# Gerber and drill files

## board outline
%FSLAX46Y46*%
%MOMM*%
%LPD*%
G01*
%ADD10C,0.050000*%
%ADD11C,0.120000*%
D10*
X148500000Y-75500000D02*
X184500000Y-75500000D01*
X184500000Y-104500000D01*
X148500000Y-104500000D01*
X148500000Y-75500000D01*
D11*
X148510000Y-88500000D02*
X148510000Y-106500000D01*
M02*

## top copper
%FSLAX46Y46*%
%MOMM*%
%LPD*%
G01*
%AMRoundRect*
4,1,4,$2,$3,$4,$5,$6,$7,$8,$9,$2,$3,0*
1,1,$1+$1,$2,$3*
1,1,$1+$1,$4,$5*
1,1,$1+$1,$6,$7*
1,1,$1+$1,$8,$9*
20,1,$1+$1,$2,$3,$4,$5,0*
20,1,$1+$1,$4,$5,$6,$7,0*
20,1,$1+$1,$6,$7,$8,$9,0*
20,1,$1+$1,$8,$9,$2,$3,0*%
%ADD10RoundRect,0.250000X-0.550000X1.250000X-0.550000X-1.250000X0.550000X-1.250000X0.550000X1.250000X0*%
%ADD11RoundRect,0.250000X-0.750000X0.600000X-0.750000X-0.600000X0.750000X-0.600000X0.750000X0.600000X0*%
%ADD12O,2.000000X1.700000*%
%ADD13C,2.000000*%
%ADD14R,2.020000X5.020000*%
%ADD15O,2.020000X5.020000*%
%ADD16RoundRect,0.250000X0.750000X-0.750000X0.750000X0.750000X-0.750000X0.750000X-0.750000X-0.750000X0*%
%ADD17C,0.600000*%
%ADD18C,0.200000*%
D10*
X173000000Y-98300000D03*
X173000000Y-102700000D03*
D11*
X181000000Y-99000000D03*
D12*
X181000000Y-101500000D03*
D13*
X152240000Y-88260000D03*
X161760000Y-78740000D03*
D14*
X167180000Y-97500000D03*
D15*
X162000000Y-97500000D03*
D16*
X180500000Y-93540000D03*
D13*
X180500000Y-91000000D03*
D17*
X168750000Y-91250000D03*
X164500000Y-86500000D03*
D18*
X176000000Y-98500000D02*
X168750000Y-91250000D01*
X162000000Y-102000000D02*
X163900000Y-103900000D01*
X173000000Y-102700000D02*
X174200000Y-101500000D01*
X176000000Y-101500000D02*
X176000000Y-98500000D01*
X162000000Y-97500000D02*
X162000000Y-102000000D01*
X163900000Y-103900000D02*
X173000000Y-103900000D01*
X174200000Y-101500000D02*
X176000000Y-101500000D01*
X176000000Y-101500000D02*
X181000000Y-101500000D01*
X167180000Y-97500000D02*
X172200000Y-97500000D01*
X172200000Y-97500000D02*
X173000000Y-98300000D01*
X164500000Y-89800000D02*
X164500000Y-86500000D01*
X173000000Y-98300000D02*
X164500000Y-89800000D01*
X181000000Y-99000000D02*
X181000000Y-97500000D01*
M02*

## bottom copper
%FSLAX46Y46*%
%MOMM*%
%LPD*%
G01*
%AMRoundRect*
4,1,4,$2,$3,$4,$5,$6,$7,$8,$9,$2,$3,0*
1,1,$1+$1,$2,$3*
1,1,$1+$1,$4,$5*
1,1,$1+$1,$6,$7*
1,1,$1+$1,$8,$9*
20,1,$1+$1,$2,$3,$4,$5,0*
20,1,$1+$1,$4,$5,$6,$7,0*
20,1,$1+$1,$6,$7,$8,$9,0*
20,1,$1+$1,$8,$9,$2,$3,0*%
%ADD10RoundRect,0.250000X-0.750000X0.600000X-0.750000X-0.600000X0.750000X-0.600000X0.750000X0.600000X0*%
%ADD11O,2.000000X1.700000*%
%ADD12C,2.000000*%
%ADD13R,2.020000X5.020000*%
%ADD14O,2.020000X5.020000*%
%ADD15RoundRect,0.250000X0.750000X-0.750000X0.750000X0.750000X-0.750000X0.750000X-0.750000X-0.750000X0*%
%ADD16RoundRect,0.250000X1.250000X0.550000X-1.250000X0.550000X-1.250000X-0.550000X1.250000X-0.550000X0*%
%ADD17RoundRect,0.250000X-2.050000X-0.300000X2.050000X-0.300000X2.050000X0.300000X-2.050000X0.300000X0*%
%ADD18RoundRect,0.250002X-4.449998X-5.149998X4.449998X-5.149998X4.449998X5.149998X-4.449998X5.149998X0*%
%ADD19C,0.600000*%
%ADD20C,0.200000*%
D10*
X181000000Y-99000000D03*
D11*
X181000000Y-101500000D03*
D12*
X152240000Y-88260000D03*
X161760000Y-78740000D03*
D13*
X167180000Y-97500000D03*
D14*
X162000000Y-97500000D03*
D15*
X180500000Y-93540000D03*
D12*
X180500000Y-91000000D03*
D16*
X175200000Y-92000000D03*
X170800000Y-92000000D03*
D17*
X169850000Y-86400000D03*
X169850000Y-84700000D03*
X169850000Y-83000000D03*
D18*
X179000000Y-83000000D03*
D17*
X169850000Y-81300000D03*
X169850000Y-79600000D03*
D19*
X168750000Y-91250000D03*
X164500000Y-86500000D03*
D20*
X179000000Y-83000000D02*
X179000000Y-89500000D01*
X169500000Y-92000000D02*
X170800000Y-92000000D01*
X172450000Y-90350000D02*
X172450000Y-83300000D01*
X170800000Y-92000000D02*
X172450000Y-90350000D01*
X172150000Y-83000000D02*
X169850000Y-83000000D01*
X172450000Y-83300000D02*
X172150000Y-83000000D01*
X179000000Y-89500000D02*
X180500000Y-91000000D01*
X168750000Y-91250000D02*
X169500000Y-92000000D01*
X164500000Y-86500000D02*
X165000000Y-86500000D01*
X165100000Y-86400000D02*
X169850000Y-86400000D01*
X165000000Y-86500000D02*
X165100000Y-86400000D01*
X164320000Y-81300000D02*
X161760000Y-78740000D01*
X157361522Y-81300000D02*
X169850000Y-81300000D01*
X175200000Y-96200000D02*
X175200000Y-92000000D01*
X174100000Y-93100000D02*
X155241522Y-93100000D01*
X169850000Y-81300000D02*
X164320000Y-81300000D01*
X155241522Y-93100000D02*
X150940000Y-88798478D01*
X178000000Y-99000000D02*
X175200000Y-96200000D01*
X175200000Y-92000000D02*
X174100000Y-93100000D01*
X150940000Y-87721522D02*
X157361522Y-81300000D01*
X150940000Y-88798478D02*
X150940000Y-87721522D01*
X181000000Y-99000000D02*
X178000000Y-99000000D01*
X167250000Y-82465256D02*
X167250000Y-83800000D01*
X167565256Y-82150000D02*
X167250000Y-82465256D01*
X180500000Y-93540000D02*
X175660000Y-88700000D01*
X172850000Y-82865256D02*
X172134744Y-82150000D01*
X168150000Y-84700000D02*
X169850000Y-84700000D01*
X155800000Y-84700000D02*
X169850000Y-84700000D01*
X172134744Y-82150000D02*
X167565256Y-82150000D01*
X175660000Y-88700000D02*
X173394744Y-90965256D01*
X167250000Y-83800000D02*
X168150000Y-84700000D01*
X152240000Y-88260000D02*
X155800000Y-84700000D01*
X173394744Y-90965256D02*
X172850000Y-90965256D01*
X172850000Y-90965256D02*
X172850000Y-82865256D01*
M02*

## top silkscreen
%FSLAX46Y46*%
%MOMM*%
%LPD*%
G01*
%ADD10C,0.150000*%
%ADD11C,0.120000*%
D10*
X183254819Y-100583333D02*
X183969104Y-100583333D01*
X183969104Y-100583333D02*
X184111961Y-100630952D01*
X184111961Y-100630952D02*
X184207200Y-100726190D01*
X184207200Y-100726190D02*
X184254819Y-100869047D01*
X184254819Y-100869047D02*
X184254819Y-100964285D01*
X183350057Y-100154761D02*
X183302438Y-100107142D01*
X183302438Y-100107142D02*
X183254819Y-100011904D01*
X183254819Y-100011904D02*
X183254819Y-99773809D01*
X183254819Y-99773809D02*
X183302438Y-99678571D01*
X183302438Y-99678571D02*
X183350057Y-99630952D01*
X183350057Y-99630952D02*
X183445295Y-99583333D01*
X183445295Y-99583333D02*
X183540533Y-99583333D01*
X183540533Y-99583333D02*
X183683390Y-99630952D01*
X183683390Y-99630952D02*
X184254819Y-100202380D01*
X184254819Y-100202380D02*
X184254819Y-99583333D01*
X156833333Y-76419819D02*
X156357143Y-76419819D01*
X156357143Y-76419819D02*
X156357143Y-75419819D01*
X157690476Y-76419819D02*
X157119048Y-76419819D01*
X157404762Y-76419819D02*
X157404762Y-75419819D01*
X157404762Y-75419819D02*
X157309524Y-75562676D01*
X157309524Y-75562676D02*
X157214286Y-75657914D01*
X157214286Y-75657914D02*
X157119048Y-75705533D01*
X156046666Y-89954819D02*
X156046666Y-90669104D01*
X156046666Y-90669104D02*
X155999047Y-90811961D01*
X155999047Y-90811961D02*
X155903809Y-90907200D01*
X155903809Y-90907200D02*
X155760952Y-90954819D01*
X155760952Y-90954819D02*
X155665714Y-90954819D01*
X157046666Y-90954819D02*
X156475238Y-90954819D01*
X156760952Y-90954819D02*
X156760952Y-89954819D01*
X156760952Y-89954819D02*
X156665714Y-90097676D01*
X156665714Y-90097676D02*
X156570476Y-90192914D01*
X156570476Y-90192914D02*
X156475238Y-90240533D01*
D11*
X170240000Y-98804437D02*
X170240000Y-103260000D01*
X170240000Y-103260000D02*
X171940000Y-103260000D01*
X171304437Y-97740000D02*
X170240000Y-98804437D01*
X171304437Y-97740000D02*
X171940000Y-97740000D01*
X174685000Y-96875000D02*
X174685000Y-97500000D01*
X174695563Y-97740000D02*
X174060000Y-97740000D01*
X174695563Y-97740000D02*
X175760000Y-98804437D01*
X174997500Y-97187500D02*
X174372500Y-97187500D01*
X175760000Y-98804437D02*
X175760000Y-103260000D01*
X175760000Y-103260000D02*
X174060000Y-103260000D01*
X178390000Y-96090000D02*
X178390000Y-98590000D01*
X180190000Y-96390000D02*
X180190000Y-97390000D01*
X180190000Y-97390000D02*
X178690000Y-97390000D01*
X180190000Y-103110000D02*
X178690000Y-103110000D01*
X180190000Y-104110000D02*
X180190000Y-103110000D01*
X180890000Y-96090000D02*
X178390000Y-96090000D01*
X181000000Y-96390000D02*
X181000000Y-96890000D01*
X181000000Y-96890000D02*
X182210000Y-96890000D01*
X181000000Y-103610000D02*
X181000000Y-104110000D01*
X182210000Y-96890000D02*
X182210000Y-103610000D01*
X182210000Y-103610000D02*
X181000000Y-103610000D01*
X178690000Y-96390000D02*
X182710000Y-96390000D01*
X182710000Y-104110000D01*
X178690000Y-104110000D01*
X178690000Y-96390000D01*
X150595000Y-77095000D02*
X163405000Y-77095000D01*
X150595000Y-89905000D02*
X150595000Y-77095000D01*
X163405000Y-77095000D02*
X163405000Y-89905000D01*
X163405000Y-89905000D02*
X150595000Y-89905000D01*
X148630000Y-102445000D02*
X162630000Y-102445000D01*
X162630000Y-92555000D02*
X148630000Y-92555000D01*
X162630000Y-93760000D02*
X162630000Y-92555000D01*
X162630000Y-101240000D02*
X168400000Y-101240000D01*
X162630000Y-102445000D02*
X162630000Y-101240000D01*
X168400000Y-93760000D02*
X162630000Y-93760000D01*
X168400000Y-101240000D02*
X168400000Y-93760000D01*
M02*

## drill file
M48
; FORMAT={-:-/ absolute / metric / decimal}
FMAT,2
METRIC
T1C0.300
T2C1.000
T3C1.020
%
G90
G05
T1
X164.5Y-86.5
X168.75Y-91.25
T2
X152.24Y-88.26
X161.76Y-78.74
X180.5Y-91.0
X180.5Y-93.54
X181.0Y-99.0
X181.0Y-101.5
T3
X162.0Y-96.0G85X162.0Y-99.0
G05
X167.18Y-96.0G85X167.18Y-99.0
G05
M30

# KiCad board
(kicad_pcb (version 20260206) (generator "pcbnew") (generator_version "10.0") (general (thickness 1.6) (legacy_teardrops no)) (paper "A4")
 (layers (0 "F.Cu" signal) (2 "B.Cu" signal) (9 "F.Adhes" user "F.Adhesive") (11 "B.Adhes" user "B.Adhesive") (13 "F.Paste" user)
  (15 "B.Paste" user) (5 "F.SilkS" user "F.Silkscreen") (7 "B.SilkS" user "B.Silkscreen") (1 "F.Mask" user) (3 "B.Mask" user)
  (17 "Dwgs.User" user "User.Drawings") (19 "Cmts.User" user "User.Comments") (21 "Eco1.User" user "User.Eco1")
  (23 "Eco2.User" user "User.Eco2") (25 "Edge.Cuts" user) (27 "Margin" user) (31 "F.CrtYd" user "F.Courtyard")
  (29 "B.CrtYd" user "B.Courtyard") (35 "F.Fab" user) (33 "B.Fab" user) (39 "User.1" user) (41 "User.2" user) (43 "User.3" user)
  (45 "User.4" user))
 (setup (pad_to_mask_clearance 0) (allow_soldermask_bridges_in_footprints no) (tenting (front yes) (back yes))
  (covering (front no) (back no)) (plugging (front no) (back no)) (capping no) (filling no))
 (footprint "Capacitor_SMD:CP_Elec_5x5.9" (layer "F.Cu") (at 173 100.5 -90)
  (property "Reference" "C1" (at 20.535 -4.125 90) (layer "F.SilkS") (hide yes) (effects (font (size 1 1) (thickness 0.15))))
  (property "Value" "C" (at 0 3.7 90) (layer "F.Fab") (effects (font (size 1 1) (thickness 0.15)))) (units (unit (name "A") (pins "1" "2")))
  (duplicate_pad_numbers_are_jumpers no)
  (fp_line (start -1.695563 2.76) (end 2.76 2.76) (stroke (width 0.12) (type solid)) (layer "F.SilkS"))
  (fp_line (start 2.76 2.76) (end 2.76 1.06) (stroke (width 0.12) (type solid)) (layer "F.SilkS"))
  (fp_line (start -2.76 1.695563) (end -1.695563 2.76) (stroke (width 0.12) (type solid)) (layer "F.SilkS"))
  (fp_line (start -2.76 1.695563) (end -2.76 1.06) (stroke (width 0.12) (type solid)) (layer "F.SilkS"))
  (fp_line (start -3.625 -1.685) (end -3 -1.685) (stroke (width 0.12) (type solid)) (layer "F.SilkS"))
  (fp_line (start -2.76 -1.695563) (end -2.76 -1.06) (stroke (width 0.12) (type solid)) (layer "F.SilkS"))
  (fp_line (start -2.76 -1.695563) (end -1.695563 -2.76) (stroke (width 0.12) (type solid)) (layer "F.SilkS"))
  (fp_line (start -3.3125 -1.9975) (end -3.3125 -1.3725) (stroke (width 0.12) (type solid)) (layer "F.SilkS"))
  (fp_line (start -1.695563 -2.76) (end 2.76 -2.76) (stroke (width 0.12) (type solid)) (layer "F.SilkS"))
  (fp_line (start 2.76 -2.76) (end 2.76 -1.06) (stroke (width 0.12) (type solid)) (layer "F.SilkS"))
  (pad "1" smd roundrect (at -2.2 0 270) (size 3 1.6) (layers "F.Cu" "F.Mask" "F.Paste") (roundrect_rratio 0.15625) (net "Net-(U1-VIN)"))
  (pad "2" smd roundrect (at 2.2 0 270) (size 3 1.6) (layers "F.Cu" "F.Mask" "F.Paste") (roundrect_rratio 0.15625) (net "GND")))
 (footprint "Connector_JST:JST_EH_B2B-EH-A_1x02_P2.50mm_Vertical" (layer "F.Cu") (at 181 99 -90)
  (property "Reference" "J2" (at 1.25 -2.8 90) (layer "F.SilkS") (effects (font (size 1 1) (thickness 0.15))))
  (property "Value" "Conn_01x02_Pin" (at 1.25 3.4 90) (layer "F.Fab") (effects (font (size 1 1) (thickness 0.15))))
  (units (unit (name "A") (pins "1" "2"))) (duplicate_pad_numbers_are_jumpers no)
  (fp_line (start -2.91 2.61) (end -0.41 2.61) (stroke (width 0.12) (type solid)) (layer "F.SilkS"))
  (fp_line (start -2.61 0.81) (end -1.61 0.81) (stroke (width 0.12) (type solid)) (layer "F.SilkS"))
  (fp_line (start -1.61 0.81) (end -1.61 2.31) (stroke (width 0.12) (type solid)) (layer "F.SilkS"))
  (fp_line (start 4.11 0.81) (end 4.11 2.31) (stroke (width 0.12) (type solid)) (layer "F.SilkS"))
  (fp_line (start 5.11 0.81) (end 4.11 0.81) (stroke (width 0.12) (type solid)) (layer "F.SilkS"))
  (fp_line (start -2.91 0.11) (end -2.91 2.61) (stroke (width 0.12) (type solid)) (layer "F.SilkS"))
  (fp_line (start -2.61 0) (end -2.11 0) (stroke (width 0.12) (type solid)) (layer "F.SilkS"))
  (fp_line (start -2.11 0) (end -2.11 -1.21) (stroke (width 0.12) (type solid)) (layer "F.SilkS"))
  (fp_line (start 4.61 0) (end 5.11 0) (stroke (width 0.12) (type solid)) (layer "F.SilkS"))
  (fp_line (start -2.11 -1.21) (end 4.61 -1.21) (stroke (width 0.12) (type solid)) (layer "F.SilkS"))
  (fp_line (start 4.61 -1.21) (end 4.61 0) (stroke (width 0.12) (type solid)) (layer "F.SilkS"))
  (fp_rect (start -2.61 -1.71) (end 5.11 2.31) (stroke (width 0.12) (type solid)) (fill no) (layer "F.SilkS"))
  (pad "1" thru_hole roundrect (at 0 0 270) (size 1.7 2) (drill 1) (layers "*.Cu" "*.Mask") (remove_unused_layers no)
   (roundrect_rratio 0.147059) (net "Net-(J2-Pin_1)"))
  (pad "2" thru_hole oval (at 2.5 0 270) (size 1.7 2) (drill 1) (layers "*.Cu" "*.Mask") (remove_unused_layers no) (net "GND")))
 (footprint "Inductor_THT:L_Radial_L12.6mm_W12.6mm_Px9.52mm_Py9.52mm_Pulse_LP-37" (layer "F.Cu") (at 152.24 88.26)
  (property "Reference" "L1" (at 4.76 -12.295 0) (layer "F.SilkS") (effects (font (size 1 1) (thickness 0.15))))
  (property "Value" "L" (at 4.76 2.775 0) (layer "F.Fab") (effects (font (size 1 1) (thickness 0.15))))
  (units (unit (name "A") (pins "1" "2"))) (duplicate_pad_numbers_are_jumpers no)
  (fp_line (start -1.645 -11.165) (end 11.165 -11.165) (stroke (width 0.12) (type solid)) (layer "F.SilkS"))
  (fp_line (start -1.645 1.645) (end -1.645 -11.165) (stroke (width 0.12) (type solid)) (layer "F.SilkS"))
  (fp_line (start 11.165 -11.165) (end 11.165 1.645) (stroke (width 0.12) (type solid)) (layer "F.SilkS"))
  (fp_line (start 11.165 1.645) (end -1.645 1.645) (stroke (width 0.12) (type solid)) (layer "F.SilkS"))
  (pad "1" thru_hole circle (at 0 0) (size 2 2) (drill 1) (layers "*.Cu" "*.Mask") (remove_unused_layers no) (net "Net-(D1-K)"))
  (pad "2" thru_hole circle (at 9.52 -9.52) (size 2 2) (drill 1) (layers "*.Cu" "*.Mask") (remove_unused_layers no) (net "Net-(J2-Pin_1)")))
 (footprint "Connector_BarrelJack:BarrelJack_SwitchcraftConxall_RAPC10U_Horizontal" (layer "F.Cu") (at 167.18 97.5)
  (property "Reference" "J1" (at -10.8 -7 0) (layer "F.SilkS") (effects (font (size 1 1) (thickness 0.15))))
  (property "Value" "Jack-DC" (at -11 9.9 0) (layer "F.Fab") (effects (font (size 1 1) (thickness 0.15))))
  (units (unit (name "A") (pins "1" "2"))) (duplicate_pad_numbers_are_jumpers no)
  (fp_line (start -18.55 4.945) (end -4.55 4.945) (stroke (width 0.12) (type solid)) (layer "F.SilkS"))
  (fp_line (start -4.55 -4.945) (end -18.55 -4.945) (stroke (width 0.12) (type solid)) (layer "F.SilkS"))
  (fp_line (start -4.55 -3.74) (end -4.55 -4.945) (stroke (width 0.12) (type solid)) (layer "F.SilkS"))
  (fp_line (start -4.55 3.74) (end 1.22 3.74) (stroke (width 0.12) (type solid)) (layer "F.SilkS"))
  (fp_line (start -4.55 4.945) (end -4.55 3.74) (stroke (width 0.12) (type solid)) (layer "F.SilkS"))
  (fp_line (start 1.22 -3.74) (end -4.55 -3.74) (stroke (width 0.12) (type solid)) (layer "F.SilkS"))
  (fp_line (start 1.22 3.74) (end 1.22 -3.74) (stroke (width 0.12) (type solid)) (layer "F.SilkS"))
  (fp_line (start -18.67 -9) (end -18.67 9) (stroke (width 0.12) (type solid)) (layer "Edge.Cuts"))
  (pad "1" thru_hole rect (at 0 0) (size 2.02 5.02) (drill oval 1.02 4.02) (layers "*.Cu" "*.Mask") (remove_unused_layers no)
   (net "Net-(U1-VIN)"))
  (pad "2" thru_hole oval (at -5.18 0) (size 2.02 5.02) (drill oval 1.02 4.02) (layers "*.Cu" "*.Mask") (remove_unused_layers no)
   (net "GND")))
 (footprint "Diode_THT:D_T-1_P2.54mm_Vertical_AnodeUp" (layer "B.Cu") (at 180.5 93.54 90)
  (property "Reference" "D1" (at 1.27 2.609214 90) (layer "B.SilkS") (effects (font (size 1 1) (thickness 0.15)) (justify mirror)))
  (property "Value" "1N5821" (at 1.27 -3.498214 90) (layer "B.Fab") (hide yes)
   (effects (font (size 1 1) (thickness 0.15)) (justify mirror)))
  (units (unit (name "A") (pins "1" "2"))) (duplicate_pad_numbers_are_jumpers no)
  (pad "1" thru_hole roundrect (at 0 0 90) (size 2 2) (drill 1) (layers "*.Cu" "*.Mask") (remove_unused_layers no) (roundrect_rratio 0.125)
   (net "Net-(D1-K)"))
  (pad "2" thru_hole circle (at 2.54 0 90) (size 2 2) (drill 1) (layers "*.Cu" "*.Mask") (remove_unused_layers no) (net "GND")))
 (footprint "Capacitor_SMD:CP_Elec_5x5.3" (layer "B.Cu") (at 173 92 180)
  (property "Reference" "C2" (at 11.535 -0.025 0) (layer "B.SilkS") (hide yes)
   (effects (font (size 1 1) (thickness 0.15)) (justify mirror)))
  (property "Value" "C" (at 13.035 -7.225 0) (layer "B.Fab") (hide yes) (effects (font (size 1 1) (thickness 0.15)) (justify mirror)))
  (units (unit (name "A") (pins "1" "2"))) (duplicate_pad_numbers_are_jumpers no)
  (pad "1" smd roundrect (at -2.2 0 180) (size 3 1.6) (layers "B.Cu" "B.Mask" "B.Paste") (roundrect_rratio 0.15625) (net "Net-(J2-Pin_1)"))
  (pad "2" smd roundrect (at 2.2 0 180) (size 3 1.6) (layers "B.Cu" "B.Mask" "B.Paste") (roundrect_rratio 0.15625) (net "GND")))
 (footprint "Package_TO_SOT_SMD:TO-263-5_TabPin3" (layer "B.Cu") (at 177.5 83)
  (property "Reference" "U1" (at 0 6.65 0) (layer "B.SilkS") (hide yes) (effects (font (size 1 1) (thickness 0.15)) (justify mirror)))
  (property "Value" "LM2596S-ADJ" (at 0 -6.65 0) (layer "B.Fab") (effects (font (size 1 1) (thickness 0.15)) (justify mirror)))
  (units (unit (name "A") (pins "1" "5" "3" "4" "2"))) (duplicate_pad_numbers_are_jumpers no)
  (pad "" smd roundrect (at -0.925 -2.775) (size 4.55 5.25) (layers "B.Paste") (roundrect_rratio 0.054945))
  (pad "" smd roundrect (at -0.925 2.775) (size 4.55 5.25) (layers "B.Paste") (roundrect_rratio 0.054945))
  (pad "" smd roundrect (at 3.925 -2.775) (size 4.55 5.25) (layers "B.Paste") (roundrect_rratio 0.054945))
  (pad "" smd roundrect (at 3.925 2.775) (size 4.55 5.25) (layers "F.Paste") (roundrect_rratio 0.054945))
  (pad "1" smd roundrect (at -7.65 3.4) (size 4.6 1.1) (layers "B.Cu" "B.Mask" "B.Paste") (roundrect_rratio 0.227273) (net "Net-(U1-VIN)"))
  (pad "2" smd roundrect (at -7.65 1.7) (size 4.6 1.1) (layers "B.Cu" "B.Mask" "B.Paste") (roundrect_rratio 0.227273) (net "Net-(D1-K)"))
  (pad "3" smd roundrect (at -7.65 0) (size 4.6 1.1) (layers "B.Cu" "B.Mask" "B.Paste") (roundrect_rratio 0.227273) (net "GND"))
  (pad "3" smd roundrect (at 1.5 0) (size 9.4 10.8) (layers "B.Cu" "B.Mask") (roundrect_rratio 0.026596) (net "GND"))
  (pad "4" smd roundrect (at -7.65 -1.7) (size 4.6 1.1) (layers "B.Cu" "B.Mask" "B.Paste") (roundrect_rratio 0.227273)
   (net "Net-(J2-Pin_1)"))
  (pad "5" smd roundrect (at -7.65 -3.4) (size 4.6 1.1) (layers "B.Cu" "B.Mask" "B.Paste") (roundrect_rratio 0.227273)
   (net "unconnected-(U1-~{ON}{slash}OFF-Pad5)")))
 (gr_rect (start 148.5 75.5) (end 184.5 104.5) (stroke (width 0.05) (type default)) (fill no) (layer "Edge.Cuts"))
 (segment (start 176 98.5) (end 168.75 91.25) (width 0.2) (layer "F.Cu") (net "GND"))
 (segment (start 162 102) (end 163.9 103.9) (width 0.2) (layer "F.Cu") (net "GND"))
 (segment (start 173 102.7) (end 174.2 101.5) (width 0.2) (layer "F.Cu") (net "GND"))
 (segment (start 176 101.5) (end 176 98.5) (width 0.2) (layer "F.Cu") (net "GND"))
 (segment (start 162 97.5) (end 162 102) (width 0.2) (layer "F.Cu") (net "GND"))
 (segment (start 163.9 103.9) (end 173 103.9) (width 0.2) (layer "F.Cu") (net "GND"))
 (segment (start 174.2 101.5) (end 176 101.5) (width 0.2) (layer "F.Cu") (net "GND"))
 (segment (start 176 101.5) (end 181 101.5) (width 0.2) (layer "F.Cu") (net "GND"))
 (via (at 168.75 91.25) (size 0.6) (drill 0.3) (layers "F.Cu" "B.Cu") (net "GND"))
 (segment (start 179 83) (end 179 89.5) (width 0.2) (layer "B.Cu") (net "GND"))
 (segment (start 169.5 92) (end 170.8 92) (width 0.2) (layer "B.Cu") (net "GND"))
 (segment (start 172.45 90.35) (end 172.45 83.3) (width 0.2) (layer "B.Cu") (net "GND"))
 (segment (start 170.8 92) (end 172.45 90.35) (width 0.2) (layer "B.Cu") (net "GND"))
 (segment (start 172.15 83) (end 169.85 83) (width 0.2) (layer "B.Cu") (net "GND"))
 (segment (start 172.45 83.3) (end 172.15 83) (width 0.2) (layer "B.Cu") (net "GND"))
 (segment (start 179 89.5) (end 180.5 91) (width 0.2) (layer "B.Cu") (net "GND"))
 (segment (start 168.75 91.25) (end 169.5 92) (width 0.2) (layer "B.Cu") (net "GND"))
 (segment (start 167.18 97.5) (end 172.2 97.5) (width 0.2) (layer "F.Cu") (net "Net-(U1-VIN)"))
 (segment (start 172.2 97.5) (end 173 98.3) (width 0.2) (layer "F.Cu") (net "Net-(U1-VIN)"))
 (segment (start 164.5 89.8) (end 164.5 86.5) (width 0.2) (layer "F.Cu") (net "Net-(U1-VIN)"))
 (segment (start 173 98.3) (end 164.5 89.8) (width 0.2) (layer "F.Cu") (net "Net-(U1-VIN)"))
 (via (at 164.5 86.5) (size 0.6) (drill 0.3) (layers "F.Cu" "B.Cu") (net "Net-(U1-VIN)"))
 (segment (start 164.5 86.5) (end 165 86.5) (width 0.2) (layer "B.Cu") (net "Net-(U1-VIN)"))
 (segment (start 165.1 86.4) (end 169.85 86.4) (width 0.2) (layer "B.Cu") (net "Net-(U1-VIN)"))
 (segment (start 165 86.5) (end 165.1 86.4) (width 0.2) (layer "B.Cu") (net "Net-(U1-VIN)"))
 (segment (start 181 99) (end 181 97.5) (width 0.2) (layer "F.Cu") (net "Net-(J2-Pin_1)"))
 (segment (start 164.32 81.3) (end 161.76 78.74) (width 0.2) (layer "B.Cu") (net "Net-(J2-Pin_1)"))
 (segment (start 157.361522 81.3) (end 169.85 81.3) (width 0.2) (layer "B.Cu") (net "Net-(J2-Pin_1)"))
 (segment (start 175.2 96.2) (end 175.2 92) (width 0.2) (layer "B.Cu") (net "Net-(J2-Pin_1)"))
 (segment (start 174.1 93.1) (end 155.241522 93.1) (width 0.2) (layer "B.Cu") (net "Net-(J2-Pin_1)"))
 (segment (start 169.85 81.3) (end 164.32 81.3) (width 0.2) (layer "B.Cu") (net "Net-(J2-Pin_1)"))
 (segment (start 155.241522 93.1) (end 150.94 88.798478) (width 0.2) (layer "B.Cu") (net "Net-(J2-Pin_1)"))
 (segment (start 178 99) (end 175.2 96.2) (width 0.2) (layer "B.Cu") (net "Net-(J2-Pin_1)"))
 (segment (start 175.2 92) (end 174.1 93.1) (width 0.2) (layer "B.Cu") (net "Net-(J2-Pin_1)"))
 (segment (start 150.94 87.721522) (end 157.361522 81.3) (width 0.2) (layer "B.Cu") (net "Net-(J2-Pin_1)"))
 (segment (start 150.94 88.798478) (end 150.94 87.721522) (width 0.2) (layer "B.Cu") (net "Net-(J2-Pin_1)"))
 (segment (start 181 99) (end 178 99) (width 0.2) (layer "B.Cu") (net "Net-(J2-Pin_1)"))
 (segment (start 167.25 82.465256) (end 167.25 83.8) (width 0.2) (layer "B.Cu") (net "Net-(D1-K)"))
 (segment (start 167.565256 82.15) (end 167.25 82.465256) (width 0.2) (layer "B.Cu") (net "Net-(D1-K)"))
 (segment (start 180.5 93.54) (end 175.66 88.7) (width 0.2) (layer "B.Cu") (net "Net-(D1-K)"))
 (segment (start 172.85 82.865256) (end 172.134744 82.15) (width 0.2) (layer "B.Cu") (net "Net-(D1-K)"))
 (segment (start 168.15 84.7) (end 169.85 84.7) (width 0.2) (layer "B.Cu") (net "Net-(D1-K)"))
 (segment (start 155.8 84.7) (end 169.85 84.7) (width 0.2) (layer "B.Cu") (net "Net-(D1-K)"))
 (segment (start 172.134744 82.15) (end 167.565256 82.15) (width 0.2) (layer "B.Cu") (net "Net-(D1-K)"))
 (segment (start 175.66 88.7) (end 173.394744 90.965256) (width 0.2) (layer "B.Cu") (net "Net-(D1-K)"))
 (segment (start 167.25 83.8) (end 168.15 84.7) (width 0.2) (layer "B.Cu") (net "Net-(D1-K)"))
 (segment (start 152.24 88.26) (end 155.8 84.7) (width 0.2) (layer "B.Cu") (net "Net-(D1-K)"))
 (segment (start 173.394744 90.965256) (end 172.85 90.965256) (width 0.2) (layer "B.Cu") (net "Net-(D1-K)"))
 (segment (start 172.85 90.965256) (end 172.85 82.865256) (width 0.2) (layer "B.Cu") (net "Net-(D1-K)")))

